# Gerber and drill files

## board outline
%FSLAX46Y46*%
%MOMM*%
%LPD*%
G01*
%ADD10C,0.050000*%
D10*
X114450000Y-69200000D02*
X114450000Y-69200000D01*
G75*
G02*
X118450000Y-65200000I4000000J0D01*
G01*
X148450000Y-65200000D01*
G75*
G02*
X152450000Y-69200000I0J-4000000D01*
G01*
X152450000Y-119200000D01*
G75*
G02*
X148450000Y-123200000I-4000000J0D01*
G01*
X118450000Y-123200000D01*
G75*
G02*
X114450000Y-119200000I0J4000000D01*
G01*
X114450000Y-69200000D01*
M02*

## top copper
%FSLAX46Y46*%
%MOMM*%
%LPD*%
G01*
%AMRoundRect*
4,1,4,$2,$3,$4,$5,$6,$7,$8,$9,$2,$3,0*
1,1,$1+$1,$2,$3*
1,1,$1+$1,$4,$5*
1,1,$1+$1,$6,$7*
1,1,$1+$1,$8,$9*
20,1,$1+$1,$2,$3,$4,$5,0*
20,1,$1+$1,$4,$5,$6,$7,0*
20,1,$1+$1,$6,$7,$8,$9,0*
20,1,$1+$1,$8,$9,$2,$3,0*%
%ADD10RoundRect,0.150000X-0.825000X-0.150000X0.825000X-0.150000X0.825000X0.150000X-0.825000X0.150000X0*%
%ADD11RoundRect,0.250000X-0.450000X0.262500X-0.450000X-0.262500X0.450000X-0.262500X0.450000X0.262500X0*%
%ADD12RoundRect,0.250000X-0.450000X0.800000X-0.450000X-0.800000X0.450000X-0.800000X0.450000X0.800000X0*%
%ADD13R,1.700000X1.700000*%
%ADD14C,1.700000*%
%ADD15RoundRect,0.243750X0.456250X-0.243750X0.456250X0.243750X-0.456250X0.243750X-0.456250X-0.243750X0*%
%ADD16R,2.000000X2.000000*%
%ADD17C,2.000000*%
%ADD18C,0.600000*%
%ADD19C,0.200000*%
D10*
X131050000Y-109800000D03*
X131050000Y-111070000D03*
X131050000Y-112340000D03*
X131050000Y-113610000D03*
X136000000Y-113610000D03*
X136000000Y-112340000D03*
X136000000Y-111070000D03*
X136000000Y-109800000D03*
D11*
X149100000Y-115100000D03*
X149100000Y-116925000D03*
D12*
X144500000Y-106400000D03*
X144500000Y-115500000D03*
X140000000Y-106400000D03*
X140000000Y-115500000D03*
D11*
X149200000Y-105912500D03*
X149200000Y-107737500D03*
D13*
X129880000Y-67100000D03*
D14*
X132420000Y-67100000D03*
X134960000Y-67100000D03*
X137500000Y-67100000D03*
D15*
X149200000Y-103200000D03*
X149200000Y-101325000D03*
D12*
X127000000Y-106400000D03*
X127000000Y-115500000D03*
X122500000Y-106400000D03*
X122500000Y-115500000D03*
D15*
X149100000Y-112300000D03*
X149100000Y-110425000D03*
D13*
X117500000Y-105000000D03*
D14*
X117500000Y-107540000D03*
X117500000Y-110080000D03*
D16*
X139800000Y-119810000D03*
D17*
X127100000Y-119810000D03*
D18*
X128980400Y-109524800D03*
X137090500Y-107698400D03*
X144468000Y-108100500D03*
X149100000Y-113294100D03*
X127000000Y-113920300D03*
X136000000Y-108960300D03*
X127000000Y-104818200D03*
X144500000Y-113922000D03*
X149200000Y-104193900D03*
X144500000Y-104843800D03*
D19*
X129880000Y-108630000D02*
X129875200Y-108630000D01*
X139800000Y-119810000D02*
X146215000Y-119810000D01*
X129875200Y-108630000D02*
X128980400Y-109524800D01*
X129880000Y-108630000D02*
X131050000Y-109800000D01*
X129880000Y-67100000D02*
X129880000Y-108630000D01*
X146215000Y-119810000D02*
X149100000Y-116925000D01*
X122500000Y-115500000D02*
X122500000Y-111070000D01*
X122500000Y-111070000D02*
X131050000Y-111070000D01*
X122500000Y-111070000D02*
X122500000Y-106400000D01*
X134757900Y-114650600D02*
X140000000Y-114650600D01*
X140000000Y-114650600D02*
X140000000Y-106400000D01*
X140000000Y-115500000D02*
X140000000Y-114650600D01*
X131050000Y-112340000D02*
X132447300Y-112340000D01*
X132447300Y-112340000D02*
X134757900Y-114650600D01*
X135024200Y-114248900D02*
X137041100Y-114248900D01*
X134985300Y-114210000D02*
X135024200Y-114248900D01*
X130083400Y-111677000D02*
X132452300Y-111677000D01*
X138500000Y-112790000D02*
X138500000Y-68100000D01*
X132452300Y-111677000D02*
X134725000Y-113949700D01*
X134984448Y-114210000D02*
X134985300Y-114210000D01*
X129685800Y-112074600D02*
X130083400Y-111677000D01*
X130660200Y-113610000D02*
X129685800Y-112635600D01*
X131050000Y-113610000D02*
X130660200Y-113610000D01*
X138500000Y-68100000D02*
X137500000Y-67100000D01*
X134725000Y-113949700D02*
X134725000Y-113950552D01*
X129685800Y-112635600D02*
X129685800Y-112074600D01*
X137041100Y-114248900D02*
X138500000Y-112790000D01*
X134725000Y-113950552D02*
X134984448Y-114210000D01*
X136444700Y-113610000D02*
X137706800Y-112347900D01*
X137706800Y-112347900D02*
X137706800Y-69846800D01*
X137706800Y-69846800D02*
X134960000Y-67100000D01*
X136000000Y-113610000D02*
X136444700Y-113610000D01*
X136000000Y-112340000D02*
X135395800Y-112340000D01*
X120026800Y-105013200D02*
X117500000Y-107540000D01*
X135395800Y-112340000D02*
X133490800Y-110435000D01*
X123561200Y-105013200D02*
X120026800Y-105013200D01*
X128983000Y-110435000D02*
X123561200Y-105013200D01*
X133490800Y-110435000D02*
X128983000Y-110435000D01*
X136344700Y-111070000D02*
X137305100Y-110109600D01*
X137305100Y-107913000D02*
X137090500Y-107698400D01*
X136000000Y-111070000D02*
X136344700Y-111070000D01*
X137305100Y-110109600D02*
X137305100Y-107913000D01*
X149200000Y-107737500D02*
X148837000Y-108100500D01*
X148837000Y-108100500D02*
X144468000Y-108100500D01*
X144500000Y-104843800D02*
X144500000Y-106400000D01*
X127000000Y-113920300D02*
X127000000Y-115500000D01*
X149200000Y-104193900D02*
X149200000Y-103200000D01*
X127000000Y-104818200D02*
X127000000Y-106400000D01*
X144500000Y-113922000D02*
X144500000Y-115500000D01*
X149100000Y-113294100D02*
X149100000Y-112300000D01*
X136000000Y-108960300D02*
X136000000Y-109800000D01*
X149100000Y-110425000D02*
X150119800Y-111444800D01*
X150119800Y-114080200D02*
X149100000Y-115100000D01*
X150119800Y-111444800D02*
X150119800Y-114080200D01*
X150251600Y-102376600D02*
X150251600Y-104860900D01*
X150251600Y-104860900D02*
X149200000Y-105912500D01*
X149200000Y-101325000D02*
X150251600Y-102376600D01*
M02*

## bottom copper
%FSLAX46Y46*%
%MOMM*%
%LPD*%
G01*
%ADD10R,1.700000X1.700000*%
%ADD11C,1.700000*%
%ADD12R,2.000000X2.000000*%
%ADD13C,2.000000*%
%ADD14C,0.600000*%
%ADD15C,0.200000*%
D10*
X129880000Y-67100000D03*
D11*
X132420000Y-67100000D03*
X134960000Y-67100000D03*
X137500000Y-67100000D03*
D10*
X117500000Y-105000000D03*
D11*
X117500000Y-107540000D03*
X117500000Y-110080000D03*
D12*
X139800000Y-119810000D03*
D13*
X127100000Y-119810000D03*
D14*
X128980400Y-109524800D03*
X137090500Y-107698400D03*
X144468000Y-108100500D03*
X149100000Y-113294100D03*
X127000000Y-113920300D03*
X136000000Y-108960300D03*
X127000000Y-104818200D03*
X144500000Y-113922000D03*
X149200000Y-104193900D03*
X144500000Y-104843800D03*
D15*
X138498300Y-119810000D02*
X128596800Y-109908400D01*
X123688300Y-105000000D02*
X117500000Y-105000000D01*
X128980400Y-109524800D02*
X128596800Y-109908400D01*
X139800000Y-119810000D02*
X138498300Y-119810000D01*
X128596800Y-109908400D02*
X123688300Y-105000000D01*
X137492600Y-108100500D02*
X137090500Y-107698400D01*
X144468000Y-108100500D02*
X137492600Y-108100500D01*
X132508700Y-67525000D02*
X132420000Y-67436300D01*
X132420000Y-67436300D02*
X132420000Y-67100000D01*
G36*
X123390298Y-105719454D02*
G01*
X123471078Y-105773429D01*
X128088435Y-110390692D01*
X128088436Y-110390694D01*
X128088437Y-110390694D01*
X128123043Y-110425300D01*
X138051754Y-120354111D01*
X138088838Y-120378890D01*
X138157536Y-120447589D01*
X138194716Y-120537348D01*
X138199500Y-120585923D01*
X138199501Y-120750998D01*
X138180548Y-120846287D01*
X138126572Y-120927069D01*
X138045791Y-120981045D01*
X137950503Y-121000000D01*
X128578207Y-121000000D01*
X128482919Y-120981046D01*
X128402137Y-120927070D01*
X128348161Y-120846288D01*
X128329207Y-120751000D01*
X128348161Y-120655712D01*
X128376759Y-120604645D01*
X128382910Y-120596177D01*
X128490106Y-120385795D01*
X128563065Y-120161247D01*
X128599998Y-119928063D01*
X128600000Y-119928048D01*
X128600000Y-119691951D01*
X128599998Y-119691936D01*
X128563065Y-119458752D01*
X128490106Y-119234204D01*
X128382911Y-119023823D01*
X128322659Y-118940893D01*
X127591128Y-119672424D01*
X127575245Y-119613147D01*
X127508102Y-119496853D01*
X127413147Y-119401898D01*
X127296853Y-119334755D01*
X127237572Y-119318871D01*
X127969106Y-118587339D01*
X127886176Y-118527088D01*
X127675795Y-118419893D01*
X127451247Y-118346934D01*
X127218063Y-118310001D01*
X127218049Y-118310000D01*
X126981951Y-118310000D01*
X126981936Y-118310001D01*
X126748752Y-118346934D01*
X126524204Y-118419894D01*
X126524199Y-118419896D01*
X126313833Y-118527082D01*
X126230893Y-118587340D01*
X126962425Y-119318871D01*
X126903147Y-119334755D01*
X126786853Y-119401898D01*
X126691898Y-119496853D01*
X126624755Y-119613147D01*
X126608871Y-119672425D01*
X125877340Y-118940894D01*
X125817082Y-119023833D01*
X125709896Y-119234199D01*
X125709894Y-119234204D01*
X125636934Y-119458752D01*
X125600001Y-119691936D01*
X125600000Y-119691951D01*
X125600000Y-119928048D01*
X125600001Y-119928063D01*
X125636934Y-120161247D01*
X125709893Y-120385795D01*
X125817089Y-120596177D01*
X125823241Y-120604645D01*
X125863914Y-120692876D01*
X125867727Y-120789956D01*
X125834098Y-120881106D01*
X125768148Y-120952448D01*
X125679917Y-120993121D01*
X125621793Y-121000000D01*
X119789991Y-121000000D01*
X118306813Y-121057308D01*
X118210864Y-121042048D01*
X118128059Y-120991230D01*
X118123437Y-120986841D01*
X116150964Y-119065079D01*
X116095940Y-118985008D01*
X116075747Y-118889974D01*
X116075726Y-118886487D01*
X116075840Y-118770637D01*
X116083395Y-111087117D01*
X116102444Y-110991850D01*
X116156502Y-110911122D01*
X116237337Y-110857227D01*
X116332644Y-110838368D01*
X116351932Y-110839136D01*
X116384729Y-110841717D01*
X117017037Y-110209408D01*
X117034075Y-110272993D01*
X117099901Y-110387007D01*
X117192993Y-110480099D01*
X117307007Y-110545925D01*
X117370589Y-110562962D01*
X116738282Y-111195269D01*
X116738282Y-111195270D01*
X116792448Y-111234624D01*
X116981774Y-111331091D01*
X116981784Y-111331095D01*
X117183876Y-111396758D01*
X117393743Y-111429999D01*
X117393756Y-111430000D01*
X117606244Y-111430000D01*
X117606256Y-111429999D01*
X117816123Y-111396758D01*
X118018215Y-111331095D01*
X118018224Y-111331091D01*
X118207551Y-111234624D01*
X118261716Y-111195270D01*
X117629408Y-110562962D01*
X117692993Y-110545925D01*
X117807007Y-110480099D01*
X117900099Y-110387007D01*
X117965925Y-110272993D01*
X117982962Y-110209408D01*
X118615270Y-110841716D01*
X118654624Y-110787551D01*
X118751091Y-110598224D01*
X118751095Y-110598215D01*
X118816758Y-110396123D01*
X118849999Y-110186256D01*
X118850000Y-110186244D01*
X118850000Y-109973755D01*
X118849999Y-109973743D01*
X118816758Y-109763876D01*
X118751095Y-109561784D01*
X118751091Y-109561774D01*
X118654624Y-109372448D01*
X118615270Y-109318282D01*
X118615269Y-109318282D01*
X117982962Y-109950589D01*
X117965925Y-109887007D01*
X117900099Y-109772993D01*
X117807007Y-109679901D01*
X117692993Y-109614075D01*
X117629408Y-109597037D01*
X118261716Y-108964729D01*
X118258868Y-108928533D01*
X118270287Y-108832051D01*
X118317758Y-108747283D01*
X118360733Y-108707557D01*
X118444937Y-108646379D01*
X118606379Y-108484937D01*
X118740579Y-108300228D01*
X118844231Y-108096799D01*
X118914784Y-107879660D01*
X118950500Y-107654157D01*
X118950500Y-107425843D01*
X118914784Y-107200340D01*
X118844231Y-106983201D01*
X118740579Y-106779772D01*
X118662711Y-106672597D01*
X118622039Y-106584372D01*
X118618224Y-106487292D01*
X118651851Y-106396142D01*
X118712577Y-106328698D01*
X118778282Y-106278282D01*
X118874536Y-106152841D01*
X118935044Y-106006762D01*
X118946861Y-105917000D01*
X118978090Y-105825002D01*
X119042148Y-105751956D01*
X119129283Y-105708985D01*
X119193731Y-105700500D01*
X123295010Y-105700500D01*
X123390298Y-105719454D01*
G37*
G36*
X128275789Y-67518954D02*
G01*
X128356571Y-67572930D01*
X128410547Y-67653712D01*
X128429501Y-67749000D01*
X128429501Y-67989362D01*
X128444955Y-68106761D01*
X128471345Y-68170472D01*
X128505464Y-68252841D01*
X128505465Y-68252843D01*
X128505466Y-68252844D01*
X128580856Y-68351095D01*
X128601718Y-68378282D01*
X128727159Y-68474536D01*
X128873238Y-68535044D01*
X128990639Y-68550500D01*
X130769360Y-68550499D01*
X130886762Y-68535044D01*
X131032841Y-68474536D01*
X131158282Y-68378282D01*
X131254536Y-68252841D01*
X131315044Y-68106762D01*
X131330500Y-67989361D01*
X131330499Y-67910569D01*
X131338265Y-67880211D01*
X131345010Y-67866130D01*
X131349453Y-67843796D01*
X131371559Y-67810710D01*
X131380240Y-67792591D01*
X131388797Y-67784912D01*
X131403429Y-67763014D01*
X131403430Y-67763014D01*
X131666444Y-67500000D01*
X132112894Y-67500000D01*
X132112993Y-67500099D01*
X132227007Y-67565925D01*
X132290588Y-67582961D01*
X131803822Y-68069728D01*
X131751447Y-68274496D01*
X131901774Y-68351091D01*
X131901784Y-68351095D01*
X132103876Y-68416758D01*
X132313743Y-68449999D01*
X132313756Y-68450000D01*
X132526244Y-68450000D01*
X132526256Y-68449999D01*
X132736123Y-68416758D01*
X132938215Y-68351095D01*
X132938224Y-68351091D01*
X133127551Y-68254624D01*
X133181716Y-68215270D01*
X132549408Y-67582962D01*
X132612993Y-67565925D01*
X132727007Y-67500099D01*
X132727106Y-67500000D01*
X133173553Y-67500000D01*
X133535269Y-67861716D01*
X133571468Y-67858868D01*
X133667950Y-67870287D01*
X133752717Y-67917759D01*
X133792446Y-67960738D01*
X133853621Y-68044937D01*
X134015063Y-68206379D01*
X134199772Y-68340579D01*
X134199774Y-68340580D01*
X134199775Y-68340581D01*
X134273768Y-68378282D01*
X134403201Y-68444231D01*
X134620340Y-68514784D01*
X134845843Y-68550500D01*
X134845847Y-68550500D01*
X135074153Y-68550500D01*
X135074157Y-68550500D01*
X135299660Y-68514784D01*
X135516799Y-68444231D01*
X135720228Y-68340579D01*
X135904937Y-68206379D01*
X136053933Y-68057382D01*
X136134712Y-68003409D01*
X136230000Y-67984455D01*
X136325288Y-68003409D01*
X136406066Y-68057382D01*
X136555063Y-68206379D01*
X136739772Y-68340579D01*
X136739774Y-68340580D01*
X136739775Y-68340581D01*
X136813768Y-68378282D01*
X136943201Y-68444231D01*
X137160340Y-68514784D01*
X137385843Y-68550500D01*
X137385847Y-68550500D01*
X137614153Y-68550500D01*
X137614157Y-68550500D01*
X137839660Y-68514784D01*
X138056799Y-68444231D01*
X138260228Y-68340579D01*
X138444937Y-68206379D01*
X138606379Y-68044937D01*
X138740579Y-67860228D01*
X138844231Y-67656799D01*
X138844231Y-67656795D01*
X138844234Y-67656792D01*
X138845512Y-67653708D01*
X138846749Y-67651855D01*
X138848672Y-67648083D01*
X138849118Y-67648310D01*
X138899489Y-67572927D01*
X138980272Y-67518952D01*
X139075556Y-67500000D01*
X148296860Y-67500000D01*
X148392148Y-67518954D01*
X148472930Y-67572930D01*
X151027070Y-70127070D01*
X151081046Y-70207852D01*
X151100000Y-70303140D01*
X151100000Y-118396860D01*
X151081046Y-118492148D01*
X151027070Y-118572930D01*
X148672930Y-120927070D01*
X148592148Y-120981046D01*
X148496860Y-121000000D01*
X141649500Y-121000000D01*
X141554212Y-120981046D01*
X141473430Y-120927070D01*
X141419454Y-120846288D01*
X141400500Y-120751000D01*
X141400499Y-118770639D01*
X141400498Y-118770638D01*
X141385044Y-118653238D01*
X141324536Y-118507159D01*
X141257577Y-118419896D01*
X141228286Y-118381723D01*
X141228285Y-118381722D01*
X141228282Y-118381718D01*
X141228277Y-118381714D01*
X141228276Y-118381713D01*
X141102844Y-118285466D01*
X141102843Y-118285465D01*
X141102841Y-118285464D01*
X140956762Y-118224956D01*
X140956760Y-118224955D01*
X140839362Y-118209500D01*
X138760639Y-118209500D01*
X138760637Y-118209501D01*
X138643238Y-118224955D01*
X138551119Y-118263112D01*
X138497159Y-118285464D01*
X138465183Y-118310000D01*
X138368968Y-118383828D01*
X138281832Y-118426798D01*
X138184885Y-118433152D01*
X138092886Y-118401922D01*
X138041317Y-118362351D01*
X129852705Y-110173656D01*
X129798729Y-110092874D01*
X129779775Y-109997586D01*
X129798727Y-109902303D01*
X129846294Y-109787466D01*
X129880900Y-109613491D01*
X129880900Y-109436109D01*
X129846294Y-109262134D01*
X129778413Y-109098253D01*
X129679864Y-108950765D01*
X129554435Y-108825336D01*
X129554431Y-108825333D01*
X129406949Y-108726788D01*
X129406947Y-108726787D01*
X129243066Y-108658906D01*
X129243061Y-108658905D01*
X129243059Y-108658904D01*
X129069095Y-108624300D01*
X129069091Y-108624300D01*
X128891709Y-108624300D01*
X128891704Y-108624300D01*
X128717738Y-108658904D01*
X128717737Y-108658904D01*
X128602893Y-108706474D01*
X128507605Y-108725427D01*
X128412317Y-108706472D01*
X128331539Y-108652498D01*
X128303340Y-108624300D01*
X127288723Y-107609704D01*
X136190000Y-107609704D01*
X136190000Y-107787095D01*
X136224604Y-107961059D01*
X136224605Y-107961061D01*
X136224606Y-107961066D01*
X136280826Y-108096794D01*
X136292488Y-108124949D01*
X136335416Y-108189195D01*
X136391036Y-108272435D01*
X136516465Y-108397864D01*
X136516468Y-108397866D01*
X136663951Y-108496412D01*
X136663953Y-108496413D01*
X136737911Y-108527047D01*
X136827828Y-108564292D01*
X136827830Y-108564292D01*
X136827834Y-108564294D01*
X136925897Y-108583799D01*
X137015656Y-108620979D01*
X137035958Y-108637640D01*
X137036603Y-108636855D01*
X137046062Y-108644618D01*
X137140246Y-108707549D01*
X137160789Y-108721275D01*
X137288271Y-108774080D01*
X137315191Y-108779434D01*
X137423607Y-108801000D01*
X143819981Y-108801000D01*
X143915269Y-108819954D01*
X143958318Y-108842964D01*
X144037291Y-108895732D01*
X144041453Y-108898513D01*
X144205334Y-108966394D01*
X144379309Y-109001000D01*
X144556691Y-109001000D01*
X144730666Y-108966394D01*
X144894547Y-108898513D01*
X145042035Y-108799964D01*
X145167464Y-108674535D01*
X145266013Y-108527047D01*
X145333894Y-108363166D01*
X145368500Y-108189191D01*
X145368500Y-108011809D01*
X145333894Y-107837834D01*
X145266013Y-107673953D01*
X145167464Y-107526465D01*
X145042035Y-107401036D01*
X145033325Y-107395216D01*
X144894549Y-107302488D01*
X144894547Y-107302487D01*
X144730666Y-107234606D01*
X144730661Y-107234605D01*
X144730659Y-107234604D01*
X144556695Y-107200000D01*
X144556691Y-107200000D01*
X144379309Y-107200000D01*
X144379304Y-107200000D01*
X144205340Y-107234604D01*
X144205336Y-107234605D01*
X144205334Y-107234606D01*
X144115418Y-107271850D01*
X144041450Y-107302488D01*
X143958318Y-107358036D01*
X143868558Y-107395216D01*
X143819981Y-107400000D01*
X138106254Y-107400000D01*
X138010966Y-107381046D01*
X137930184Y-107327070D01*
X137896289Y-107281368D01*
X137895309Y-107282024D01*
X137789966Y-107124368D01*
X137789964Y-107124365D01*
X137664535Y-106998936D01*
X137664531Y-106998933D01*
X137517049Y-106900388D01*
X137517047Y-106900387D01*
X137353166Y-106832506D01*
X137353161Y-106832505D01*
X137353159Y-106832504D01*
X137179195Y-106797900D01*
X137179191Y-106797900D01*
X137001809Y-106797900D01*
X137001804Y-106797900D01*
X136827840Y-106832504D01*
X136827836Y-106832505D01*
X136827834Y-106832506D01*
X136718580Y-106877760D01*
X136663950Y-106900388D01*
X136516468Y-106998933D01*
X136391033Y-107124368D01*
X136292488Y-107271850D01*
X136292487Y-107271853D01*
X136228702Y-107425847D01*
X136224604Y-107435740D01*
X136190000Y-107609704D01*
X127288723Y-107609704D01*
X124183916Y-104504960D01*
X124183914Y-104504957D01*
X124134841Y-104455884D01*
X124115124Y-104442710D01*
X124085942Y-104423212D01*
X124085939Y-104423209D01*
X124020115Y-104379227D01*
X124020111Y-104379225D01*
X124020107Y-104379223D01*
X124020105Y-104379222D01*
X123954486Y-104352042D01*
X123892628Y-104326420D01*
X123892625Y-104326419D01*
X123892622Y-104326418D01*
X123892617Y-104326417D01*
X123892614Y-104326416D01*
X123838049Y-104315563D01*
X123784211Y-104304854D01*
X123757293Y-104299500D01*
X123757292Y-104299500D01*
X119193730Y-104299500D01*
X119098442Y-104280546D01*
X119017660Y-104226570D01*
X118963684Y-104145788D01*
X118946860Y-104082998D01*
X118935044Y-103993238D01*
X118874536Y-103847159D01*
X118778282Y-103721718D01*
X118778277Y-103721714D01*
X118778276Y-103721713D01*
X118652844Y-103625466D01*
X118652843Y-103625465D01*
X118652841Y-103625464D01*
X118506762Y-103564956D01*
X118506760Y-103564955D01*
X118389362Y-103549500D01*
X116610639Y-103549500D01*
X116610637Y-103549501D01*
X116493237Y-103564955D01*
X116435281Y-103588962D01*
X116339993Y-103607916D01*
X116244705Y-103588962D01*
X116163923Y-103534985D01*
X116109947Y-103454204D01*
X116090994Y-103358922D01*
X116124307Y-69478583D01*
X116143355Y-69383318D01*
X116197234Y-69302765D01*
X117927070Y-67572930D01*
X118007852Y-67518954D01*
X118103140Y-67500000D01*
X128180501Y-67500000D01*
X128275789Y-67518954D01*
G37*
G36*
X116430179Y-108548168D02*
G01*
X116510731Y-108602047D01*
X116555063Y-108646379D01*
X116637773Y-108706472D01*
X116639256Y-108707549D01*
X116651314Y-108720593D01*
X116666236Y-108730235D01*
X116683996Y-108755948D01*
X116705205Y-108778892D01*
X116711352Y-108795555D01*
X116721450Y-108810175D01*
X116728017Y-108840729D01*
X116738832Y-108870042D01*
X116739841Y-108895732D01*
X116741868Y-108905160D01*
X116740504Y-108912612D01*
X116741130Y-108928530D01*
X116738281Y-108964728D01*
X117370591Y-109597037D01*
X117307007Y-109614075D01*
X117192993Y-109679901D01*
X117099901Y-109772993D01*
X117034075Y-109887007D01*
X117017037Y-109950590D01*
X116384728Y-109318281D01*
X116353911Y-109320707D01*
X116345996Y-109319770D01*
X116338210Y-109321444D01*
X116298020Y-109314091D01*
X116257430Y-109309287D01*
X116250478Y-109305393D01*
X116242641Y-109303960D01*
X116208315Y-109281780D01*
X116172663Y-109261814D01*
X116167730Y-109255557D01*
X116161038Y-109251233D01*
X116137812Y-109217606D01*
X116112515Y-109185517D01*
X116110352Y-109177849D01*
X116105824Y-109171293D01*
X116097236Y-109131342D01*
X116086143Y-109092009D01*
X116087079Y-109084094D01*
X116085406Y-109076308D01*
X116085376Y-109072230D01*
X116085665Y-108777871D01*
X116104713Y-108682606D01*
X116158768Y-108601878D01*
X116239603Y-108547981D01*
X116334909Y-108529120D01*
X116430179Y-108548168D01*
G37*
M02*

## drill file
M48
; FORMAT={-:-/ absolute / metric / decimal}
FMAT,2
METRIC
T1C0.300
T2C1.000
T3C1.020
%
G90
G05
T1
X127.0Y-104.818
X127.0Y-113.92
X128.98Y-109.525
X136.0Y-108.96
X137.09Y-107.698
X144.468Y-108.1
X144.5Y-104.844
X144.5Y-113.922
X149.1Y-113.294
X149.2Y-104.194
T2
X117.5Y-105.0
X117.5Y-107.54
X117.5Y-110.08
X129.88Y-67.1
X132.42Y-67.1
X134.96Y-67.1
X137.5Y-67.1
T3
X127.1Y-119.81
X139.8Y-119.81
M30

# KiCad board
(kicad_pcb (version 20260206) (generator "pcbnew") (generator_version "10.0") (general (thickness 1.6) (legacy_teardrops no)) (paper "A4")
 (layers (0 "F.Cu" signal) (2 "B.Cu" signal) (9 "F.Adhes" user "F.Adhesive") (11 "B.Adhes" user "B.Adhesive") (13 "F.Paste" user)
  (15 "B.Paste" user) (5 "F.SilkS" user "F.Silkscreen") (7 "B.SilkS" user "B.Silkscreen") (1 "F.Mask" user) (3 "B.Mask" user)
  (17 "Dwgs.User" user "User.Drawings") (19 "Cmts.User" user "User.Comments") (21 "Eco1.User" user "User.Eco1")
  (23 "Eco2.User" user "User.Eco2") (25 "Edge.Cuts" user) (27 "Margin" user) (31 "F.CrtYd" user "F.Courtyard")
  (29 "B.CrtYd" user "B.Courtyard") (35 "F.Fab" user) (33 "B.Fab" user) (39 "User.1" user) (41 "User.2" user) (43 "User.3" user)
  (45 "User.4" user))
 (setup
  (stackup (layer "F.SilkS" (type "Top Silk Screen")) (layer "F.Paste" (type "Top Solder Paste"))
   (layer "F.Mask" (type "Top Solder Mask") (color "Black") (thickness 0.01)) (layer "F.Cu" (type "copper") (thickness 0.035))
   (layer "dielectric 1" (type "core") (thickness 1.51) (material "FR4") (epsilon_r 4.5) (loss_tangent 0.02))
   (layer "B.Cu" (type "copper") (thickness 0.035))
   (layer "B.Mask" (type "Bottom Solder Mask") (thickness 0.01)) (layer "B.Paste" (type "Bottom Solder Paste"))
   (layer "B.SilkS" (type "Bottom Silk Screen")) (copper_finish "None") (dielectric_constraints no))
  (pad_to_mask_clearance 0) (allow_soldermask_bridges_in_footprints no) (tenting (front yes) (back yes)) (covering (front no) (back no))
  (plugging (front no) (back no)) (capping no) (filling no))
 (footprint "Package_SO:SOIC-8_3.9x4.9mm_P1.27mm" (layer "F.Cu") (at 133.525 111.705)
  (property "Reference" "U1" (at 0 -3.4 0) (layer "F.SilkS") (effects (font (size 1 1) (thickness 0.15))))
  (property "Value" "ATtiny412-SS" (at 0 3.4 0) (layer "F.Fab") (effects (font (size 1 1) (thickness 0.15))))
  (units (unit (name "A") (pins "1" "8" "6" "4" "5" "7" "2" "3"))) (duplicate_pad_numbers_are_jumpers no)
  (pad "1" smd roundrect (at -2.475 -1.905) (size 1.95 0.6) (layers "F.Cu" "F.Mask" "F.Paste") (roundrect_rratio 0.25) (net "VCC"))
  (pad "2" smd roundrect (at -2.475 -0.635) (size 1.95 0.6) (layers "F.Cu" "F.Mask" "F.Paste") (roundrect_rratio 0.25) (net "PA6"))
  (pad "3" smd roundrect (at -2.475 0.635) (size 1.95 0.6) (layers "F.Cu" "F.Mask" "F.Paste") (roundrect_rratio 0.25) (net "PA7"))
  (pad "4" smd roundrect (at -2.475 1.905) (size 1.95 0.6) (layers "F.Cu" "F.Mask" "F.Paste") (roundrect_rratio 0.25) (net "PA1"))
  (pad "5" smd roundrect (at 2.475 1.905) (size 1.95 0.6) (layers "F.Cu" "F.Mask" "F.Paste") (roundrect_rratio 0.25) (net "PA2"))
  (pad "6" smd roundrect (at 2.475 0.635) (size 1.95 0.6) (layers "F.Cu" "F.Mask" "F.Paste") (roundrect_rratio 0.25)
   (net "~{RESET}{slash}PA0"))
  (pad "7" smd roundrect (at 2.475 -0.635) (size 1.95 0.6) (layers "F.Cu" "F.Mask" "F.Paste") (roundrect_rratio 0.25) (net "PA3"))
  (pad "8" smd roundrect (at 2.475 -1.905) (size 1.95 0.6) (layers "F.Cu" "F.Mask" "F.Paste") (roundrect_rratio 0.25) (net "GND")))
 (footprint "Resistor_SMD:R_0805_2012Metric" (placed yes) (layer "F.Cu") (at 149.1 116.0125 -90)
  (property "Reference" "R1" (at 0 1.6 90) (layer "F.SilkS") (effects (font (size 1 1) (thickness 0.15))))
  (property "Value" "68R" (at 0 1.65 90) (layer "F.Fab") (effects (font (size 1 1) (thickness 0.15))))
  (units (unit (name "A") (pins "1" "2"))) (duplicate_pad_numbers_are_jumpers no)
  (pad "1" smd roundrect (at -0.9125 0 270) (size 1.025 1.4) (layers "F.Cu" "F.Mask" "F.Paste") (roundrect_rratio 0.243902)
   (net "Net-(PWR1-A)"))
  (pad "2" smd roundrect (at 0.9125 0 270) (size 1.025 1.4) (layers "F.Cu" "F.Mask" "F.Paste") (roundrect_rratio 0.243902) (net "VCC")))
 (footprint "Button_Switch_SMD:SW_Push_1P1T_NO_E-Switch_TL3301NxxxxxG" (layer "F.Cu") (at 142.25 110.95 -90)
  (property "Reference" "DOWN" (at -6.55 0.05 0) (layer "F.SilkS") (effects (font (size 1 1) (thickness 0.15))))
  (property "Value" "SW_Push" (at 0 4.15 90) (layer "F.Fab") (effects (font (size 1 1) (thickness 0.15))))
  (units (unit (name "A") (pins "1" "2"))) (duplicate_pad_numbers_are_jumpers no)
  (pad "1" smd roundrect (at -4.55 -2.25 270) (size 2.1 1.4) (layers "F.Cu" "F.Mask" "F.Paste") (roundrect_rratio 0.1785714286) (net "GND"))
  (pad "1" smd roundrect (at 4.55 -2.25 270) (size 2.1 1.4) (layers "F.Cu" "F.Mask" "F.Paste") (roundrect_rratio 0.1785714286) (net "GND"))
  (pad "2" smd roundrect (at -4.55 2.25 270) (size 2.1 1.4) (layers "F.Cu" "F.Mask" "F.Paste") (roundrect_rratio 0.1785714286) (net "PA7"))
  (pad "2" smd roundrect (at 4.55 2.25 270) (size 2.1 1.4) (layers "F.Cu" "F.Mask" "F.Paste") (roundrect_rratio 0.1785714286) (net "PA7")))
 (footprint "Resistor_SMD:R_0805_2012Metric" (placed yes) (layer "F.Cu") (at 149.2 106.825 -90)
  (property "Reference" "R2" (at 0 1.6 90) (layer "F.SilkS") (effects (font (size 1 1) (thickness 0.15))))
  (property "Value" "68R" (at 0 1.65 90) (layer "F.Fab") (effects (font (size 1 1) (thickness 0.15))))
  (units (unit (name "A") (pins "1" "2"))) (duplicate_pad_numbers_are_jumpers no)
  (pad "1" smd roundrect (at -0.9125 0 270) (size 1.025 1.4) (layers "F.Cu" "F.Mask" "F.Paste") (roundrect_rratio 0.243902)
   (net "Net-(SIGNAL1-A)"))
  (pad "2" smd roundrect (at 0.9125 0 270) (size 1.025 1.4) (layers "F.Cu" "F.Mask" "F.Paste") (roundrect_rratio 0.243902) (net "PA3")))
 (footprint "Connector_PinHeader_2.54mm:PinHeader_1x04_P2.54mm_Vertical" (layer "F.Cu") (at 129.88 67.1 90)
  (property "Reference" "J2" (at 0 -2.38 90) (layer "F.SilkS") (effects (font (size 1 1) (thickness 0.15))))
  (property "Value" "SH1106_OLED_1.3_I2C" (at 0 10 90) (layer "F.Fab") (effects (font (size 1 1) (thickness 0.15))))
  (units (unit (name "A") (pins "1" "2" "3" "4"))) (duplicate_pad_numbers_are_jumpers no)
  (pad "1" thru_hole rect (at 0 0 90) (size 1.7 1.7) (drill 1) (layers "*.Cu" "*.Mask") (remove_unused_layers no) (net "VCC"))
  (pad "2" thru_hole circle (at 0 2.54 90) (size 1.7 1.7) (drill 1) (layers "*.Cu" "*.Mask") (remove_unused_layers no) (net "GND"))
  (pad "3" thru_hole circle (at 0 5.08 90) (size 1.7 1.7) (drill 1) (layers "*.Cu" "*.Mask") (remove_unused_layers no) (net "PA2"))
  (pad "4" thru_hole circle (at 0 7.62 90) (size 1.7 1.7) (drill 1) (layers "*.Cu" "*.Mask") (remove_unused_layers no) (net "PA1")))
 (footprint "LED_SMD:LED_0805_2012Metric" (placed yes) (layer "F.Cu") (at 149.2 102.2625 90)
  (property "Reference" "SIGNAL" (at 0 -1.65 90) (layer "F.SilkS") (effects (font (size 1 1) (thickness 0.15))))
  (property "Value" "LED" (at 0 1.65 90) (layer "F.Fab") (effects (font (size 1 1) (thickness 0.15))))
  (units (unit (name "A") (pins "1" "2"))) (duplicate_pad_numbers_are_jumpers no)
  (pad "1" smd roundrect (at -0.9375 0 90) (size 0.975 1.4) (layers "F.Cu" "F.Mask" "F.Paste") (roundrect_rratio 0.25) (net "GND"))
  (pad "2" smd roundrect (at 0.9375 0 90) (size 0.975 1.4) (layers "F.Cu" "F.Mask" "F.Paste") (roundrect_rratio 0.25)
   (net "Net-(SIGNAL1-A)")))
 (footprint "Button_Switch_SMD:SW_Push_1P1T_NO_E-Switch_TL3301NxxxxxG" (layer "F.Cu") (at 124.75 110.95 -90)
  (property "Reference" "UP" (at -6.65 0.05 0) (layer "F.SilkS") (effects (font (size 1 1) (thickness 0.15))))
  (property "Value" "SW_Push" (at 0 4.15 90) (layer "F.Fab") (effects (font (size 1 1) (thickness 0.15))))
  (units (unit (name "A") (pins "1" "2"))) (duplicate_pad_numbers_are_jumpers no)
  (pad "1" smd roundrect (at -4.55 -2.25 270) (size 2.1 1.4) (layers "F.Cu" "F.Mask" "F.Paste") (roundrect_rratio 0.1785714286) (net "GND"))
  (pad "1" smd roundrect (at 4.55 -2.25 270) (size 2.1 1.4) (layers "F.Cu" "F.Mask" "F.Paste") (roundrect_rratio 0.1785714286) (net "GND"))
  (pad "2" smd roundrect (at -4.55 2.25 270) (size 2.1 1.4) (layers "F.Cu" "F.Mask" "F.Paste") (roundrect_rratio 0.1785714286) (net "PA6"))
  (pad "2" smd roundrect (at 4.55 2.25 270) (size 2.1 1.4) (layers "F.Cu" "F.Mask" "F.Paste") (roundrect_rratio 0.1785714286) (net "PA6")))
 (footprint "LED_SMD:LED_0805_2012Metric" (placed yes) (layer "F.Cu") (at 149.1 111.3625 90)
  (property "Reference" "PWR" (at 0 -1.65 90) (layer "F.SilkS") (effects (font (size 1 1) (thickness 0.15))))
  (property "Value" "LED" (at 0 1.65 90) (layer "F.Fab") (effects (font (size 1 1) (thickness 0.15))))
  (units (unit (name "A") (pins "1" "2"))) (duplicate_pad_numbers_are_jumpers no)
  (pad "1" smd roundrect (at -0.9375 0 90) (size 0.975 1.4) (layers "F.Cu" "F.Mask" "F.Paste") (roundrect_rratio 0.25) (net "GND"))
  (pad "2" smd roundrect (at 0.9375 0 90) (size 0.975 1.4) (layers "F.Cu" "F.Mask" "F.Paste") (roundrect_rratio 0.25) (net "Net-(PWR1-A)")))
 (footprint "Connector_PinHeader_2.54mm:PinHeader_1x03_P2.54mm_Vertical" (layer "F.Cu") (at 117.5 105)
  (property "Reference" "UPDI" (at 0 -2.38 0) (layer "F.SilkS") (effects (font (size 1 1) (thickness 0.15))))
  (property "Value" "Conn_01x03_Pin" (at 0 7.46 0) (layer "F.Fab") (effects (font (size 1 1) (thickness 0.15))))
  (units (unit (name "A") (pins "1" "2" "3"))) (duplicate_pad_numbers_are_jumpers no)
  (pad "1" thru_hole rect (at 0 0) (size 1.7 1.7) (drill 1) (layers "*.Cu" "*.Mask") (remove_unused_layers no) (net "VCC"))
  (pad "2" thru_hole circle (at 0 2.54) (size 1.7 1.7) (drill 1) (layers "*.Cu" "*.Mask") (remove_unused_layers no)
   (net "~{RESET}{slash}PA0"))
  (pad "3" thru_hole circle (at 0 5.08) (size 1.7 1.7) (drill 1) (layers "*.Cu" "*.Mask") (remove_unused_layers no) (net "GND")))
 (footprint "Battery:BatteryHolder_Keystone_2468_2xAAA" (layer "B.Cu") (at 139.8 119.81 90)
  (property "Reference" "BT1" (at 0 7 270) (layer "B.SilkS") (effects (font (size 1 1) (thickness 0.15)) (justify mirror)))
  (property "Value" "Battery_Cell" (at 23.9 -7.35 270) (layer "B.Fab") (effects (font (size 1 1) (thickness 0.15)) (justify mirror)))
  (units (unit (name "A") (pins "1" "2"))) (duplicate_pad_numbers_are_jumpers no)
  (pad "1" thru_hole rect (at 0 0 90) (size 2 2) (drill 1.02) (layers "*.Cu" "*.Mask") (remove_unused_layers no) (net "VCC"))
  (pad "2" thru_hole circle (at 0 -12.7 90) (size 2 2) (drill 1.02) (layers "*.Cu" "*.Mask") (remove_unused_layers no) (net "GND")))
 (gr_rect (start 114.45 65.2) (end 152.45 123.2) (radius 4) (stroke (width 0.05) (type solid)) (fill no) (layer "Edge.Cuts"))
 (segment (start 129.88 108.63) (end 129.8752 108.63) (width 0.2) (layer "F.Cu") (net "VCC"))
 (segment (start 139.8 119.81) (end 146.215 119.81) (width 0.2) (layer "F.Cu") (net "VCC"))
 (segment (start 129.8752 108.63) (end 128.9804 109.5248) (width 0.2) (layer "F.Cu") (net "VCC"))
 (segment (start 129.88 108.63) (end 131.05 109.8) (width 0.2) (layer "F.Cu") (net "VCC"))
 (segment (start 129.88 67.1) (end 129.88 108.63) (width 0.2) (layer "F.Cu") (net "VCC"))
 (segment (start 146.215 119.81) (end 149.1 116.925) (width 0.2) (layer "F.Cu") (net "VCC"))
 (via (at 128.9804 109.5248) (size 0.6) (drill 0.3) (layers "F.Cu" "B.Cu") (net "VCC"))
 (segment (start 138.4983 119.81) (end 128.5968 109.9084) (width 0.2) (layer "B.Cu") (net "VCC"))
 (segment (start 123.6883 105) (end 117.5 105) (width 0.2) (layer "B.Cu") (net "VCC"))
 (segment (start 128.9804 109.5248) (end 128.5968 109.9084) (width 0.2) (layer "B.Cu") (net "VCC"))
 (segment (start 139.8 119.81) (end 138.4983 119.81) (width 0.2) (layer "B.Cu") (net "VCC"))
 (segment (start 128.5968 109.9084) (end 123.6883 105) (width 0.2) (layer "B.Cu") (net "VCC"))
 (segment (start 122.5 115.5) (end 122.5 111.07) (width 0.2) (layer "F.Cu") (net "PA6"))
 (segment (start 122.5 111.07) (end 131.05 111.07) (width 0.2) (layer "F.Cu") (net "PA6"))
 (segment (start 122.5 111.07) (end 122.5 106.4) (width 0.2) (layer "F.Cu") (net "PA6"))
 (segment (start 134.7579 114.6506) (end 140 114.6506) (width 0.2) (layer "F.Cu") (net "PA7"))
 (segment (start 140 114.6506) (end 140 106.4) (width 0.2) (layer "F.Cu") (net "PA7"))
 (segment (start 140 115.5) (end 140 114.6506) (width 0.2) (layer "F.Cu") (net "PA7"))
 (segment (start 131.05 112.34) (end 132.4473 112.34) (width 0.2) (layer "F.Cu") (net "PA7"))
 (segment (start 132.4473 112.34) (end 134.7579 114.6506) (width 0.2) (layer "F.Cu") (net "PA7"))
 (segment (start 135.0242 114.2489) (end 137.0411 114.2489) (width 0.2) (layer "F.Cu") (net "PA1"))
 (segment (start 134.9853 114.21) (end 135.0242 114.2489) (width 0.2) (layer "F.Cu") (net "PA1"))
 (segment (start 130.0834 111.677) (end 132.4523 111.677) (width 0.2) (layer "F.Cu") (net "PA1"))
 (segment (start 138.5 112.79) (end 138.5 68.1) (width 0.2) (layer "F.Cu") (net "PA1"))
 (segment (start 132.4523 111.677) (end 134.725 113.9497) (width 0.2) (layer "F.Cu") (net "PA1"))
 (segment (start 134.984448 114.21) (end 134.9853 114.21) (width 0.2) (layer "F.Cu") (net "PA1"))
 (segment (start 129.6858 112.0746) (end 130.0834 111.677) (width 0.2) (layer "F.Cu") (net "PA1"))
 (segment (start 130.6602 113.61) (end 129.6858 112.6356) (width 0.2) (layer "F.Cu") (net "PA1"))
 (segment (start 131.05 113.61) (end 130.6602 113.61) (width 0.2) (layer "F.Cu") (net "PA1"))
 (segment (start 138.5 68.1) (end 137.5 67.1) (width 0.2) (layer "F.Cu") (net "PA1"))
 (segment (start 134.725 113.9497) (end 134.725 113.950552) (width 0.2) (layer "F.Cu") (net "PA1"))
 (segment (start 129.6858 112.6356) (end 129.6858 112.0746) (width 0.2) (layer "F.Cu") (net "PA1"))
 (segment (start 137.0411 114.2489) (end 138.5 112.79) (width 0.2) (layer "F.Cu") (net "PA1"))
 (segment (start 134.725 113.950552) (end 134.984448 114.21) (width 0.2) (layer "F.Cu") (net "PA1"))
 (segment (start 136.4447 113.61) (end 137.7068 112.3479) (width 0.2) (layer "F.Cu") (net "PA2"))
 (segment (start 137.7068 112.3479) (end 137.7068 69.8468) (width 0.2) (layer "F.Cu") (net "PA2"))
 (segment (start 137.7068 69.8468) (end 134.96 67.1) (width 0.2) (layer "F.Cu") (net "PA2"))
 (segment (start 136 113.61) (end 136.4447 113.61) (width 0.2) (layer "F.Cu") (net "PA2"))
 (segment (start 136 112.34) (end 135.3958 112.34) (width 0.2) (layer "F.Cu") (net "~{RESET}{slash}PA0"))
 (segment (start 120.0268 105.0132) (end 117.5 107.54) (width 0.2) (layer "F.Cu") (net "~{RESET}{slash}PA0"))
 (segment (start 135.3958 112.34) (end 133.4908 110.435) (width 0.2) (layer "F.Cu") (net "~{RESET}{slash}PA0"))
 (segment (start 123.5612 105.0132) (end 120.0268 105.0132) (width 0.2) (layer "F.Cu") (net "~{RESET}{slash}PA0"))
 (segment (start 128.983 110.435) (end 123.5612 105.0132) (width 0.2) (layer "F.Cu") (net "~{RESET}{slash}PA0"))
 (segment (start 133.4908 110.435) (end 128.983 110.435) (width 0.2) (layer "F.Cu") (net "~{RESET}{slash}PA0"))
 (segment (start 136.3447 111.07) (end 137.3051 110.1096) (width 0.2) (layer "F.Cu") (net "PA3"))
 (segment (start 137.3051 107.913) (end 137.0905 107.6984) (width 0.2) (layer "F.Cu") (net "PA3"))
 (segment (start 136 111.07) (end 136.3447 111.07) (width 0.2) (layer "F.Cu") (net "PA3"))
 (segment (start 137.3051 110.1096) (end 137.3051 107.913) (width 0.2) (layer "F.Cu") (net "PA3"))
 (segment (start 149.2 107.7375) (end 148.837 108.1005) (width 0.2) (layer "F.Cu") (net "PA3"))
 (segment (start 148.837 108.1005) (end 144.468 108.1005) (width 0.2) (layer "F.Cu") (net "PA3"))
 (via (at 137.0905 107.6984) (size 0.6) (drill 0.3) (layers "F.Cu" "B.Cu") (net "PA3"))
 (via (at 144.468 108.1005) (size 0.6) (drill 0.3) (layers "F.Cu" "B.Cu") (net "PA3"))
 (segment (start 137.4926 108.1005) (end 137.0905 107.6984) (width 0.2) (layer "B.Cu") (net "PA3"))
 (segment (start 144.468 108.1005) (end 137.4926 108.1005) (width 0.2) (layer "B.Cu") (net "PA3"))
 (segment (start 144.5 104.8438) (end 144.5 106.4) (width 0.2) (layer "F.Cu") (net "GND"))
 (segment (start 127 113.9203) (end 127 115.5) (width 0.2) (layer "F.Cu") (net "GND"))
 (segment (start 149.2 104.1939) (end 149.2 103.2) (width 0.2) (layer "F.Cu") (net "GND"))
 (segment (start 127 104.8182) (end 127 106.4) (width 0.2) (layer "F.Cu") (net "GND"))
 (segment (start 144.5 113.922) (end 144.5 115.5) (width 0.2) (layer "F.Cu") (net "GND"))
 (segment (start 149.1 113.2941) (end 149.1 112.3) (width 0.2) (layer "F.Cu") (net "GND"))
 (segment (start 136 108.9603) (end 136 109.8) (width 0.2) (layer "F.Cu") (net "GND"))
 (via (at 149.1 113.2941) (size 0.6) (drill 0.3) (layers "F.Cu" "B.Cu") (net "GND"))
 (via (at 127 113.9203) (size 0.6) (drill 0.3) (layers "F.Cu" "B.Cu") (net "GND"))
 (via (at 136 108.9603) (size 0.6) (drill 0.3) (layers "F.Cu" "B.Cu") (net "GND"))
 (via (at 127 104.8182) (size 0.6) (drill 0.3) (layers "F.Cu" "B.Cu") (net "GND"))
 (via (at 144.5 113.922) (size 0.6) (drill 0.3) (layers "F.Cu" "B.Cu") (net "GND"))
 (via (at 149.2 104.1939) (size 0.6) (drill 0.3) (layers "F.Cu" "B.Cu") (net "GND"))
 (via (at 144.5 104.8438) (size 0.6) (drill 0.3) (layers "F.Cu" "B.Cu") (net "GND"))
 (segment (start 132.5087 67.525) (end 132.42 67.4363) (width 0.2) (layer "B.Cu") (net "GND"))
 (segment (start 132.42 67.4363) (end 132.42 67.1) (width 0.2) (layer "B.Cu") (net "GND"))
 (segment (start 149.1 110.425) (end 150.1198 111.4448) (width 0.2) (layer "F.Cu") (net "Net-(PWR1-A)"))
 (segment (start 150.1198 114.0802) (end 149.1 115.1) (width 0.2) (layer "F.Cu") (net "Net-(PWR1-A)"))
 (segment (start 150.1198 111.4448) (end 150.1198 114.0802) (width 0.2) (layer "F.Cu") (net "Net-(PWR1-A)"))
 (segment (start 150.2516 102.3766) (end 150.2516 104.8609) (width 0.2) (layer "F.Cu") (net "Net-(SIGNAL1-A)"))
 (segment (start 150.2516 104.8609) (end 149.2 105.9125) (width 0.2) (layer "F.Cu") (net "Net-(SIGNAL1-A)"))
 (segment (start 149.2 101.325) (end 150.2516 102.3766) (width 0.2) (layer "F.Cu") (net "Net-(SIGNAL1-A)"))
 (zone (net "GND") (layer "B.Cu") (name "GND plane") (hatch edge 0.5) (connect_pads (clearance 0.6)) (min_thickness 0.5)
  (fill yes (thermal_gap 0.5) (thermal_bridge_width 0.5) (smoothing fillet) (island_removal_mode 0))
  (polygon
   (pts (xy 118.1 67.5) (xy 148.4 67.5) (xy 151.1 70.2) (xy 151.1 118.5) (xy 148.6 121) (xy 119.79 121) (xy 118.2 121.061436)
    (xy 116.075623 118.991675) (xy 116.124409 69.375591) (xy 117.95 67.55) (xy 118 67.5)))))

